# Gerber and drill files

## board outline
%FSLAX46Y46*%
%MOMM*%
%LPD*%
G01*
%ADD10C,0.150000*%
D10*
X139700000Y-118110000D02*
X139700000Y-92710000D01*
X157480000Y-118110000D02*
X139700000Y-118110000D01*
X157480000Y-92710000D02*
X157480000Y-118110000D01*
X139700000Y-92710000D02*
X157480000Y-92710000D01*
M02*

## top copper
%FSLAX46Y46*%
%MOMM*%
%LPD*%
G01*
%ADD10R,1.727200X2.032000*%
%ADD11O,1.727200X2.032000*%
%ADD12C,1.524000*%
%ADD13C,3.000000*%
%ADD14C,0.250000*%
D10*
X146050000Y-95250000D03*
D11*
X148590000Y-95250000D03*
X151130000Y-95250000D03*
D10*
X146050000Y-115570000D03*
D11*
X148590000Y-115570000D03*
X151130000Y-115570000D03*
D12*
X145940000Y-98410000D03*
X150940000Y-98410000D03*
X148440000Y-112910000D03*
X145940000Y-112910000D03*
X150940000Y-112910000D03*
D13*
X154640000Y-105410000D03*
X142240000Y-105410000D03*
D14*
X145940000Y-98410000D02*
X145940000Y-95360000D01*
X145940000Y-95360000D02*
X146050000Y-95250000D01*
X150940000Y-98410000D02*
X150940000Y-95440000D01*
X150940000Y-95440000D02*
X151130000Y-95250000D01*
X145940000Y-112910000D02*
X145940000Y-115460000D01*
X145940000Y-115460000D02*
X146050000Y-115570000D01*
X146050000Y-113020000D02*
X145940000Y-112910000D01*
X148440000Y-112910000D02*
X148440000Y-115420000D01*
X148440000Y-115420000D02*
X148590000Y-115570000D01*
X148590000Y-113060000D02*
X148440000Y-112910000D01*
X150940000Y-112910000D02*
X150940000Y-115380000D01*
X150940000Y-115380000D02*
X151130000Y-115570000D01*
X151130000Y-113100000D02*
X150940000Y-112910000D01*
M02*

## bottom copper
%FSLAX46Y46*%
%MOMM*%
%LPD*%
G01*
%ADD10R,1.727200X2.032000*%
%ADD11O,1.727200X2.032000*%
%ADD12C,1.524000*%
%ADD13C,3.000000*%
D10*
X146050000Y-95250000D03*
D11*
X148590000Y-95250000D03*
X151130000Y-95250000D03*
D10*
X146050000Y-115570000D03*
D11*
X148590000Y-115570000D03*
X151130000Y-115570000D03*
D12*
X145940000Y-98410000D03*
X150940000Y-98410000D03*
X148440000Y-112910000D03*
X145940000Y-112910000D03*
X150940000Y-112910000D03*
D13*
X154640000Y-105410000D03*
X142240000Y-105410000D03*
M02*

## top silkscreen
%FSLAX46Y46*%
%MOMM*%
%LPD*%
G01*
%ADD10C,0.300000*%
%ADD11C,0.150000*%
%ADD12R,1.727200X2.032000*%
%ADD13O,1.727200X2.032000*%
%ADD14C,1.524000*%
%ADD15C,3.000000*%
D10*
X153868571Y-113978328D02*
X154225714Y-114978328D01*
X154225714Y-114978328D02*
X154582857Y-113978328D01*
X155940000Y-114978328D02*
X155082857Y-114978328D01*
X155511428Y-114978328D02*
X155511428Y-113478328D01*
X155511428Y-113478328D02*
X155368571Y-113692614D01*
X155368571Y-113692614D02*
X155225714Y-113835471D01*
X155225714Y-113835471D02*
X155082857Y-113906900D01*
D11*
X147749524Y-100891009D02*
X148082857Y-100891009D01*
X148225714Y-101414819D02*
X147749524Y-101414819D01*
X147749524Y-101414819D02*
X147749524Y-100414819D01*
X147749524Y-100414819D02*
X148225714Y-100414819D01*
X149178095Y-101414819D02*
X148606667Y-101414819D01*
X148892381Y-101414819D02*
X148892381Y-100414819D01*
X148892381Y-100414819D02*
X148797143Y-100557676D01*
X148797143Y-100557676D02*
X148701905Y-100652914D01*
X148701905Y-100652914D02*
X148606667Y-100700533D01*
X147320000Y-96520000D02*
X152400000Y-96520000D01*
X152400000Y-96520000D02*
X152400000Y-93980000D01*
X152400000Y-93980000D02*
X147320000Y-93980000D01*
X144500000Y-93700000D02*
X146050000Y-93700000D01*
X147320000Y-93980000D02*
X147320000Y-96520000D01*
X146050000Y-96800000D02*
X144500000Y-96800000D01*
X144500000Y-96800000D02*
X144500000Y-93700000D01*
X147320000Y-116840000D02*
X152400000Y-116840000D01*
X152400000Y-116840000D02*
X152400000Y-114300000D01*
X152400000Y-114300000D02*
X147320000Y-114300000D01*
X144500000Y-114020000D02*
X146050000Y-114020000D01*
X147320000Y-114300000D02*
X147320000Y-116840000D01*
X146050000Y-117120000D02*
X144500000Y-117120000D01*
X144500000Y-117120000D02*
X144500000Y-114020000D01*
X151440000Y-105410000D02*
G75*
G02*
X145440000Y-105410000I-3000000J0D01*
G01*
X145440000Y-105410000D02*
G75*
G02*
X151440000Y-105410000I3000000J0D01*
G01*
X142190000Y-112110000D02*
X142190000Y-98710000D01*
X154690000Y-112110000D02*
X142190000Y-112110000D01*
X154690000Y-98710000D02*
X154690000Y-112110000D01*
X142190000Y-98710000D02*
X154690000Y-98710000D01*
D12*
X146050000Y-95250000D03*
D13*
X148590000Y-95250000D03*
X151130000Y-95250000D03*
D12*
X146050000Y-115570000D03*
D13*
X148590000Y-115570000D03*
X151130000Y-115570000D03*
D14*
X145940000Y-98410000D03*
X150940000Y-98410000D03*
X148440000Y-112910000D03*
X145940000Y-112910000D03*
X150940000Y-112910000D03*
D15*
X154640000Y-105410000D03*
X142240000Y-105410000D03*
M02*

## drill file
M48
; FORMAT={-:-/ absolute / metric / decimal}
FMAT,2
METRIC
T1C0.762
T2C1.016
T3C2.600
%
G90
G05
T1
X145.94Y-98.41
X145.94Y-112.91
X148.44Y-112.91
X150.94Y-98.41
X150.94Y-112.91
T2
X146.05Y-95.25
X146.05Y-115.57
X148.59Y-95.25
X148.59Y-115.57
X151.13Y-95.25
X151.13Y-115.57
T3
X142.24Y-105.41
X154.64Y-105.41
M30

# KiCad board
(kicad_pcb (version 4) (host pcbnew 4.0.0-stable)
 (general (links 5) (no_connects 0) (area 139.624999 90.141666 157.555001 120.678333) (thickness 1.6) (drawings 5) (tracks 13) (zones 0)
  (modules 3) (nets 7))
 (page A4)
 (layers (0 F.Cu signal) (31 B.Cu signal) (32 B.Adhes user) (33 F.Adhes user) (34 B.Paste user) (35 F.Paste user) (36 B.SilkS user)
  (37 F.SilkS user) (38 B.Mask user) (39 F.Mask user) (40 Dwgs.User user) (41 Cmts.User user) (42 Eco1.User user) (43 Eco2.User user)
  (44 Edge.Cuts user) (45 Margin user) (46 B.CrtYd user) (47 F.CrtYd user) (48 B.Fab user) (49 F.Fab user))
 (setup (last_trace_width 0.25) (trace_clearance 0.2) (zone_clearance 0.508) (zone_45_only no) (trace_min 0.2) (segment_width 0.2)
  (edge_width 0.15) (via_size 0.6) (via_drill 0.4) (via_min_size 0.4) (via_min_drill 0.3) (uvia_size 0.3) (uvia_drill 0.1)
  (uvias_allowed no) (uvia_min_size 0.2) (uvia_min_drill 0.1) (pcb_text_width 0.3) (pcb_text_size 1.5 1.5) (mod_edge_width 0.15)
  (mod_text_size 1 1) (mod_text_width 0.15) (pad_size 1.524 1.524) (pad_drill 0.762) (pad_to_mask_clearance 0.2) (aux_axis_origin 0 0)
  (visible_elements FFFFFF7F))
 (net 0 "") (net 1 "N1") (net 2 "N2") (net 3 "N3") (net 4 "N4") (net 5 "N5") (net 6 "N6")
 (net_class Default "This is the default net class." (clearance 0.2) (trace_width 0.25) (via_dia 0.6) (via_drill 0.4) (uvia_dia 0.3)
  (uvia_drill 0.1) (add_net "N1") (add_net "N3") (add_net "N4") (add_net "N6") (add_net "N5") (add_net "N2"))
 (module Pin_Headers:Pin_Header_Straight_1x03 (layer F.Cu) (at 146.05 95.25 90)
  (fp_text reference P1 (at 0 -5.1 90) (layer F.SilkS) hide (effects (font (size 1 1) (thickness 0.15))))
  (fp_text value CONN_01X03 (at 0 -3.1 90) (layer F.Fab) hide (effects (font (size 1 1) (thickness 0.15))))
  (fp_line (start -1.27 1.27) (end -1.27 6.35) (layer F.SilkS) (width 0.15))
  (fp_line (start -1.27 6.35) (end 1.27 6.35) (layer F.SilkS) (width 0.15))
  (fp_line (start 1.27 6.35) (end 1.27 1.27) (layer F.SilkS) (width 0.15))
  (fp_line (start 1.55 -1.55) (end 1.55 0) (layer F.SilkS) (width 0.15))
  (fp_line (start 1.27 1.27) (end -1.27 1.27) (layer F.SilkS) (width 0.15))
  (fp_line (start -1.55 0) (end -1.55 -1.55) (layer F.SilkS) (width 0.15))
  (fp_line (start -1.55 -1.55) (end 1.55 -1.55) (layer F.SilkS) (width 0.15))
  (pad 1 thru_hole rect (at 0 0 90) (size 2.032 1.7272) (drill 1.016) (layers *.Cu *.Mask F.SilkS) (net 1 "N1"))
  (pad 2 thru_hole oval (at 0 2.54 90) (size 2.032 1.7272) (drill 1.016) (layers *.Cu *.Mask F.SilkS) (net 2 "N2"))
  (pad 3 thru_hole oval (at 0 5.08 90) (size 2.032 1.7272) (drill 1.016) (layers *.Cu *.Mask F.SilkS) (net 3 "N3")))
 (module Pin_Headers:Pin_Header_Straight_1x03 (layer F.Cu) (at 146.05 115.57 90)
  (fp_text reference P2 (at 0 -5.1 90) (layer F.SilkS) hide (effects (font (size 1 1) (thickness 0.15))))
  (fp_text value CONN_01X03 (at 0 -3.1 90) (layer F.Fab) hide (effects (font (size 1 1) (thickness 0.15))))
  (fp_line (start -1.27 1.27) (end -1.27 6.35) (layer F.SilkS) (width 0.15))
  (fp_line (start -1.27 6.35) (end 1.27 6.35) (layer F.SilkS) (width 0.15))
  (fp_line (start 1.27 6.35) (end 1.27 1.27) (layer F.SilkS) (width 0.15))
  (fp_line (start 1.55 -1.55) (end 1.55 0) (layer F.SilkS) (width 0.15))
  (fp_line (start 1.27 1.27) (end -1.27 1.27) (layer F.SilkS) (width 0.15))
  (fp_line (start -1.55 0) (end -1.55 -1.55) (layer F.SilkS) (width 0.15))
  (fp_line (start -1.55 -1.55) (end 1.55 -1.55) (layer F.SilkS) (width 0.15))
  (pad 1 thru_hole rect (at 0 0 90) (size 2.032 1.7272) (drill 1.016) (layers *.Cu *.Mask F.SilkS) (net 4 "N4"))
  (pad 2 thru_hole oval (at 0 2.54 90) (size 2.032 1.7272) (drill 1.016) (layers *.Cu *.Mask F.SilkS) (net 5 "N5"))
  (pad 3 thru_hole oval (at 0 5.08 90) (size 2.032 1.7272) (drill 1.016) (layers *.Cu *.Mask F.SilkS) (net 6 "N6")))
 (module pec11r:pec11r (layer F.Cu) (at 148.44 105.41)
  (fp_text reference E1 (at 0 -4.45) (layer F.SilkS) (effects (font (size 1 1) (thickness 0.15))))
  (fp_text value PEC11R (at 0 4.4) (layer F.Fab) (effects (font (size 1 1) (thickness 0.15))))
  (fp_circle (center 0 0) (end 3 0) (layer F.SilkS) (width 0.15))
  (fp_line (start -6.25 6.7) (end -6.25 -6.7) (layer F.SilkS) (width 0.15))
  (fp_line (start 6.25 6.7) (end -6.25 6.7) (layer F.SilkS) (width 0.15))
  (fp_line (start 6.25 -6.7) (end 6.25 6.7) (layer F.SilkS) (width 0.15))
  (fp_line (start -6.25 -6.7) (end 6.25 -6.7) (layer F.SilkS) (width 0.15))
  (pad 1 thru_hole circle (at -2.5 -7) (size 1.524 1.524) (drill 0.762) (layers *.Cu *.Mask F.SilkS) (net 1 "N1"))
  (pad 2 thru_hole circle (at 2.5 -7) (size 1.524 1.524) (drill 0.762) (layers *.Cu *.Mask F.SilkS) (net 3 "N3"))
  (pad C thru_hole circle (at 0 7.5) (size 1.524 1.524) (drill 0.762) (layers *.Cu *.Mask F.SilkS) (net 5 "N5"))
  (pad A thru_hole circle (at -2.5 7.5) (size 1.524 1.524) (drill 0.762) (layers *.Cu *.Mask F.SilkS) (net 4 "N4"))
  (pad B thru_hole circle (at 2.5 7.5) (size 1.524 1.524) (drill 0.762) (layers *.Cu *.Mask F.SilkS) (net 6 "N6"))
  (pad "" thru_hole circle (at 6.2 0) (size 3 3) (drill 2.6) (layers *.Cu *.Mask F.SilkS))
  (pad "" thru_hole circle (at -6.2 0) (size 3 3) (drill 2.6) (layers *.Cu *.Mask F.SilkS)))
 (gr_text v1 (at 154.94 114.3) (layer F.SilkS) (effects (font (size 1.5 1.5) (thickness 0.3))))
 (gr_line (start 139.7 118.11) (end 139.7 92.71) (layer Edge.Cuts) (width 0.15))
 (gr_line (start 157.48 118.11) (end 139.7 118.11) (layer Edge.Cuts) (width 0.15))
 (gr_line (start 157.48 92.71) (end 157.48 118.11) (layer Edge.Cuts) (width 0.15))
 (gr_line (start 139.7 92.71) (end 157.48 92.71) (layer Edge.Cuts) (width 0.15))
 (segment (start 145.94 98.41) (end 145.94 95.36) (width 0.25) (layer F.Cu) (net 1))
 (segment (start 145.94 95.36) (end 146.05 95.25) (width 0.25) (layer F.Cu) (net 1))
 (segment (start 150.94 98.41) (end 150.94 95.44) (width 0.25) (layer F.Cu) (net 3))
 (segment (start 150.94 95.44) (end 151.13 95.25) (width 0.25) (layer F.Cu) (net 3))
 (segment (start 145.94 112.91) (end 145.94 115.46) (width 0.25) (layer F.Cu) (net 4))
 (segment (start 145.94 115.46) (end 146.05 115.57) (width 0.25) (layer F.Cu) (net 4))
 (segment (start 146.05 113.02) (end 145.94 112.91) (width 0.25) (layer F.Cu) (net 4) (status 30))
 (segment (start 148.44 112.91) (end 148.44 115.42) (width 0.25) (layer F.Cu) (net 5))
 (segment (start 148.44 115.42) (end 148.59 115.57) (width 0.25) (layer F.Cu) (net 5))
 (segment (start 148.59 113.06) (end 148.44 112.91) (width 0.25) (layer F.Cu) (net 5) (status 30))
 (segment (start 150.94 112.91) (end 150.94 115.38) (width 0.25) (layer F.Cu) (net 6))
 (segment (start 150.94 115.38) (end 151.13 115.57) (width 0.25) (layer F.Cu) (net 6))
 (segment (start 151.13 113.1) (end 150.94 112.91) (width 0.25) (layer F.Cu) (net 6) (status 30)))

